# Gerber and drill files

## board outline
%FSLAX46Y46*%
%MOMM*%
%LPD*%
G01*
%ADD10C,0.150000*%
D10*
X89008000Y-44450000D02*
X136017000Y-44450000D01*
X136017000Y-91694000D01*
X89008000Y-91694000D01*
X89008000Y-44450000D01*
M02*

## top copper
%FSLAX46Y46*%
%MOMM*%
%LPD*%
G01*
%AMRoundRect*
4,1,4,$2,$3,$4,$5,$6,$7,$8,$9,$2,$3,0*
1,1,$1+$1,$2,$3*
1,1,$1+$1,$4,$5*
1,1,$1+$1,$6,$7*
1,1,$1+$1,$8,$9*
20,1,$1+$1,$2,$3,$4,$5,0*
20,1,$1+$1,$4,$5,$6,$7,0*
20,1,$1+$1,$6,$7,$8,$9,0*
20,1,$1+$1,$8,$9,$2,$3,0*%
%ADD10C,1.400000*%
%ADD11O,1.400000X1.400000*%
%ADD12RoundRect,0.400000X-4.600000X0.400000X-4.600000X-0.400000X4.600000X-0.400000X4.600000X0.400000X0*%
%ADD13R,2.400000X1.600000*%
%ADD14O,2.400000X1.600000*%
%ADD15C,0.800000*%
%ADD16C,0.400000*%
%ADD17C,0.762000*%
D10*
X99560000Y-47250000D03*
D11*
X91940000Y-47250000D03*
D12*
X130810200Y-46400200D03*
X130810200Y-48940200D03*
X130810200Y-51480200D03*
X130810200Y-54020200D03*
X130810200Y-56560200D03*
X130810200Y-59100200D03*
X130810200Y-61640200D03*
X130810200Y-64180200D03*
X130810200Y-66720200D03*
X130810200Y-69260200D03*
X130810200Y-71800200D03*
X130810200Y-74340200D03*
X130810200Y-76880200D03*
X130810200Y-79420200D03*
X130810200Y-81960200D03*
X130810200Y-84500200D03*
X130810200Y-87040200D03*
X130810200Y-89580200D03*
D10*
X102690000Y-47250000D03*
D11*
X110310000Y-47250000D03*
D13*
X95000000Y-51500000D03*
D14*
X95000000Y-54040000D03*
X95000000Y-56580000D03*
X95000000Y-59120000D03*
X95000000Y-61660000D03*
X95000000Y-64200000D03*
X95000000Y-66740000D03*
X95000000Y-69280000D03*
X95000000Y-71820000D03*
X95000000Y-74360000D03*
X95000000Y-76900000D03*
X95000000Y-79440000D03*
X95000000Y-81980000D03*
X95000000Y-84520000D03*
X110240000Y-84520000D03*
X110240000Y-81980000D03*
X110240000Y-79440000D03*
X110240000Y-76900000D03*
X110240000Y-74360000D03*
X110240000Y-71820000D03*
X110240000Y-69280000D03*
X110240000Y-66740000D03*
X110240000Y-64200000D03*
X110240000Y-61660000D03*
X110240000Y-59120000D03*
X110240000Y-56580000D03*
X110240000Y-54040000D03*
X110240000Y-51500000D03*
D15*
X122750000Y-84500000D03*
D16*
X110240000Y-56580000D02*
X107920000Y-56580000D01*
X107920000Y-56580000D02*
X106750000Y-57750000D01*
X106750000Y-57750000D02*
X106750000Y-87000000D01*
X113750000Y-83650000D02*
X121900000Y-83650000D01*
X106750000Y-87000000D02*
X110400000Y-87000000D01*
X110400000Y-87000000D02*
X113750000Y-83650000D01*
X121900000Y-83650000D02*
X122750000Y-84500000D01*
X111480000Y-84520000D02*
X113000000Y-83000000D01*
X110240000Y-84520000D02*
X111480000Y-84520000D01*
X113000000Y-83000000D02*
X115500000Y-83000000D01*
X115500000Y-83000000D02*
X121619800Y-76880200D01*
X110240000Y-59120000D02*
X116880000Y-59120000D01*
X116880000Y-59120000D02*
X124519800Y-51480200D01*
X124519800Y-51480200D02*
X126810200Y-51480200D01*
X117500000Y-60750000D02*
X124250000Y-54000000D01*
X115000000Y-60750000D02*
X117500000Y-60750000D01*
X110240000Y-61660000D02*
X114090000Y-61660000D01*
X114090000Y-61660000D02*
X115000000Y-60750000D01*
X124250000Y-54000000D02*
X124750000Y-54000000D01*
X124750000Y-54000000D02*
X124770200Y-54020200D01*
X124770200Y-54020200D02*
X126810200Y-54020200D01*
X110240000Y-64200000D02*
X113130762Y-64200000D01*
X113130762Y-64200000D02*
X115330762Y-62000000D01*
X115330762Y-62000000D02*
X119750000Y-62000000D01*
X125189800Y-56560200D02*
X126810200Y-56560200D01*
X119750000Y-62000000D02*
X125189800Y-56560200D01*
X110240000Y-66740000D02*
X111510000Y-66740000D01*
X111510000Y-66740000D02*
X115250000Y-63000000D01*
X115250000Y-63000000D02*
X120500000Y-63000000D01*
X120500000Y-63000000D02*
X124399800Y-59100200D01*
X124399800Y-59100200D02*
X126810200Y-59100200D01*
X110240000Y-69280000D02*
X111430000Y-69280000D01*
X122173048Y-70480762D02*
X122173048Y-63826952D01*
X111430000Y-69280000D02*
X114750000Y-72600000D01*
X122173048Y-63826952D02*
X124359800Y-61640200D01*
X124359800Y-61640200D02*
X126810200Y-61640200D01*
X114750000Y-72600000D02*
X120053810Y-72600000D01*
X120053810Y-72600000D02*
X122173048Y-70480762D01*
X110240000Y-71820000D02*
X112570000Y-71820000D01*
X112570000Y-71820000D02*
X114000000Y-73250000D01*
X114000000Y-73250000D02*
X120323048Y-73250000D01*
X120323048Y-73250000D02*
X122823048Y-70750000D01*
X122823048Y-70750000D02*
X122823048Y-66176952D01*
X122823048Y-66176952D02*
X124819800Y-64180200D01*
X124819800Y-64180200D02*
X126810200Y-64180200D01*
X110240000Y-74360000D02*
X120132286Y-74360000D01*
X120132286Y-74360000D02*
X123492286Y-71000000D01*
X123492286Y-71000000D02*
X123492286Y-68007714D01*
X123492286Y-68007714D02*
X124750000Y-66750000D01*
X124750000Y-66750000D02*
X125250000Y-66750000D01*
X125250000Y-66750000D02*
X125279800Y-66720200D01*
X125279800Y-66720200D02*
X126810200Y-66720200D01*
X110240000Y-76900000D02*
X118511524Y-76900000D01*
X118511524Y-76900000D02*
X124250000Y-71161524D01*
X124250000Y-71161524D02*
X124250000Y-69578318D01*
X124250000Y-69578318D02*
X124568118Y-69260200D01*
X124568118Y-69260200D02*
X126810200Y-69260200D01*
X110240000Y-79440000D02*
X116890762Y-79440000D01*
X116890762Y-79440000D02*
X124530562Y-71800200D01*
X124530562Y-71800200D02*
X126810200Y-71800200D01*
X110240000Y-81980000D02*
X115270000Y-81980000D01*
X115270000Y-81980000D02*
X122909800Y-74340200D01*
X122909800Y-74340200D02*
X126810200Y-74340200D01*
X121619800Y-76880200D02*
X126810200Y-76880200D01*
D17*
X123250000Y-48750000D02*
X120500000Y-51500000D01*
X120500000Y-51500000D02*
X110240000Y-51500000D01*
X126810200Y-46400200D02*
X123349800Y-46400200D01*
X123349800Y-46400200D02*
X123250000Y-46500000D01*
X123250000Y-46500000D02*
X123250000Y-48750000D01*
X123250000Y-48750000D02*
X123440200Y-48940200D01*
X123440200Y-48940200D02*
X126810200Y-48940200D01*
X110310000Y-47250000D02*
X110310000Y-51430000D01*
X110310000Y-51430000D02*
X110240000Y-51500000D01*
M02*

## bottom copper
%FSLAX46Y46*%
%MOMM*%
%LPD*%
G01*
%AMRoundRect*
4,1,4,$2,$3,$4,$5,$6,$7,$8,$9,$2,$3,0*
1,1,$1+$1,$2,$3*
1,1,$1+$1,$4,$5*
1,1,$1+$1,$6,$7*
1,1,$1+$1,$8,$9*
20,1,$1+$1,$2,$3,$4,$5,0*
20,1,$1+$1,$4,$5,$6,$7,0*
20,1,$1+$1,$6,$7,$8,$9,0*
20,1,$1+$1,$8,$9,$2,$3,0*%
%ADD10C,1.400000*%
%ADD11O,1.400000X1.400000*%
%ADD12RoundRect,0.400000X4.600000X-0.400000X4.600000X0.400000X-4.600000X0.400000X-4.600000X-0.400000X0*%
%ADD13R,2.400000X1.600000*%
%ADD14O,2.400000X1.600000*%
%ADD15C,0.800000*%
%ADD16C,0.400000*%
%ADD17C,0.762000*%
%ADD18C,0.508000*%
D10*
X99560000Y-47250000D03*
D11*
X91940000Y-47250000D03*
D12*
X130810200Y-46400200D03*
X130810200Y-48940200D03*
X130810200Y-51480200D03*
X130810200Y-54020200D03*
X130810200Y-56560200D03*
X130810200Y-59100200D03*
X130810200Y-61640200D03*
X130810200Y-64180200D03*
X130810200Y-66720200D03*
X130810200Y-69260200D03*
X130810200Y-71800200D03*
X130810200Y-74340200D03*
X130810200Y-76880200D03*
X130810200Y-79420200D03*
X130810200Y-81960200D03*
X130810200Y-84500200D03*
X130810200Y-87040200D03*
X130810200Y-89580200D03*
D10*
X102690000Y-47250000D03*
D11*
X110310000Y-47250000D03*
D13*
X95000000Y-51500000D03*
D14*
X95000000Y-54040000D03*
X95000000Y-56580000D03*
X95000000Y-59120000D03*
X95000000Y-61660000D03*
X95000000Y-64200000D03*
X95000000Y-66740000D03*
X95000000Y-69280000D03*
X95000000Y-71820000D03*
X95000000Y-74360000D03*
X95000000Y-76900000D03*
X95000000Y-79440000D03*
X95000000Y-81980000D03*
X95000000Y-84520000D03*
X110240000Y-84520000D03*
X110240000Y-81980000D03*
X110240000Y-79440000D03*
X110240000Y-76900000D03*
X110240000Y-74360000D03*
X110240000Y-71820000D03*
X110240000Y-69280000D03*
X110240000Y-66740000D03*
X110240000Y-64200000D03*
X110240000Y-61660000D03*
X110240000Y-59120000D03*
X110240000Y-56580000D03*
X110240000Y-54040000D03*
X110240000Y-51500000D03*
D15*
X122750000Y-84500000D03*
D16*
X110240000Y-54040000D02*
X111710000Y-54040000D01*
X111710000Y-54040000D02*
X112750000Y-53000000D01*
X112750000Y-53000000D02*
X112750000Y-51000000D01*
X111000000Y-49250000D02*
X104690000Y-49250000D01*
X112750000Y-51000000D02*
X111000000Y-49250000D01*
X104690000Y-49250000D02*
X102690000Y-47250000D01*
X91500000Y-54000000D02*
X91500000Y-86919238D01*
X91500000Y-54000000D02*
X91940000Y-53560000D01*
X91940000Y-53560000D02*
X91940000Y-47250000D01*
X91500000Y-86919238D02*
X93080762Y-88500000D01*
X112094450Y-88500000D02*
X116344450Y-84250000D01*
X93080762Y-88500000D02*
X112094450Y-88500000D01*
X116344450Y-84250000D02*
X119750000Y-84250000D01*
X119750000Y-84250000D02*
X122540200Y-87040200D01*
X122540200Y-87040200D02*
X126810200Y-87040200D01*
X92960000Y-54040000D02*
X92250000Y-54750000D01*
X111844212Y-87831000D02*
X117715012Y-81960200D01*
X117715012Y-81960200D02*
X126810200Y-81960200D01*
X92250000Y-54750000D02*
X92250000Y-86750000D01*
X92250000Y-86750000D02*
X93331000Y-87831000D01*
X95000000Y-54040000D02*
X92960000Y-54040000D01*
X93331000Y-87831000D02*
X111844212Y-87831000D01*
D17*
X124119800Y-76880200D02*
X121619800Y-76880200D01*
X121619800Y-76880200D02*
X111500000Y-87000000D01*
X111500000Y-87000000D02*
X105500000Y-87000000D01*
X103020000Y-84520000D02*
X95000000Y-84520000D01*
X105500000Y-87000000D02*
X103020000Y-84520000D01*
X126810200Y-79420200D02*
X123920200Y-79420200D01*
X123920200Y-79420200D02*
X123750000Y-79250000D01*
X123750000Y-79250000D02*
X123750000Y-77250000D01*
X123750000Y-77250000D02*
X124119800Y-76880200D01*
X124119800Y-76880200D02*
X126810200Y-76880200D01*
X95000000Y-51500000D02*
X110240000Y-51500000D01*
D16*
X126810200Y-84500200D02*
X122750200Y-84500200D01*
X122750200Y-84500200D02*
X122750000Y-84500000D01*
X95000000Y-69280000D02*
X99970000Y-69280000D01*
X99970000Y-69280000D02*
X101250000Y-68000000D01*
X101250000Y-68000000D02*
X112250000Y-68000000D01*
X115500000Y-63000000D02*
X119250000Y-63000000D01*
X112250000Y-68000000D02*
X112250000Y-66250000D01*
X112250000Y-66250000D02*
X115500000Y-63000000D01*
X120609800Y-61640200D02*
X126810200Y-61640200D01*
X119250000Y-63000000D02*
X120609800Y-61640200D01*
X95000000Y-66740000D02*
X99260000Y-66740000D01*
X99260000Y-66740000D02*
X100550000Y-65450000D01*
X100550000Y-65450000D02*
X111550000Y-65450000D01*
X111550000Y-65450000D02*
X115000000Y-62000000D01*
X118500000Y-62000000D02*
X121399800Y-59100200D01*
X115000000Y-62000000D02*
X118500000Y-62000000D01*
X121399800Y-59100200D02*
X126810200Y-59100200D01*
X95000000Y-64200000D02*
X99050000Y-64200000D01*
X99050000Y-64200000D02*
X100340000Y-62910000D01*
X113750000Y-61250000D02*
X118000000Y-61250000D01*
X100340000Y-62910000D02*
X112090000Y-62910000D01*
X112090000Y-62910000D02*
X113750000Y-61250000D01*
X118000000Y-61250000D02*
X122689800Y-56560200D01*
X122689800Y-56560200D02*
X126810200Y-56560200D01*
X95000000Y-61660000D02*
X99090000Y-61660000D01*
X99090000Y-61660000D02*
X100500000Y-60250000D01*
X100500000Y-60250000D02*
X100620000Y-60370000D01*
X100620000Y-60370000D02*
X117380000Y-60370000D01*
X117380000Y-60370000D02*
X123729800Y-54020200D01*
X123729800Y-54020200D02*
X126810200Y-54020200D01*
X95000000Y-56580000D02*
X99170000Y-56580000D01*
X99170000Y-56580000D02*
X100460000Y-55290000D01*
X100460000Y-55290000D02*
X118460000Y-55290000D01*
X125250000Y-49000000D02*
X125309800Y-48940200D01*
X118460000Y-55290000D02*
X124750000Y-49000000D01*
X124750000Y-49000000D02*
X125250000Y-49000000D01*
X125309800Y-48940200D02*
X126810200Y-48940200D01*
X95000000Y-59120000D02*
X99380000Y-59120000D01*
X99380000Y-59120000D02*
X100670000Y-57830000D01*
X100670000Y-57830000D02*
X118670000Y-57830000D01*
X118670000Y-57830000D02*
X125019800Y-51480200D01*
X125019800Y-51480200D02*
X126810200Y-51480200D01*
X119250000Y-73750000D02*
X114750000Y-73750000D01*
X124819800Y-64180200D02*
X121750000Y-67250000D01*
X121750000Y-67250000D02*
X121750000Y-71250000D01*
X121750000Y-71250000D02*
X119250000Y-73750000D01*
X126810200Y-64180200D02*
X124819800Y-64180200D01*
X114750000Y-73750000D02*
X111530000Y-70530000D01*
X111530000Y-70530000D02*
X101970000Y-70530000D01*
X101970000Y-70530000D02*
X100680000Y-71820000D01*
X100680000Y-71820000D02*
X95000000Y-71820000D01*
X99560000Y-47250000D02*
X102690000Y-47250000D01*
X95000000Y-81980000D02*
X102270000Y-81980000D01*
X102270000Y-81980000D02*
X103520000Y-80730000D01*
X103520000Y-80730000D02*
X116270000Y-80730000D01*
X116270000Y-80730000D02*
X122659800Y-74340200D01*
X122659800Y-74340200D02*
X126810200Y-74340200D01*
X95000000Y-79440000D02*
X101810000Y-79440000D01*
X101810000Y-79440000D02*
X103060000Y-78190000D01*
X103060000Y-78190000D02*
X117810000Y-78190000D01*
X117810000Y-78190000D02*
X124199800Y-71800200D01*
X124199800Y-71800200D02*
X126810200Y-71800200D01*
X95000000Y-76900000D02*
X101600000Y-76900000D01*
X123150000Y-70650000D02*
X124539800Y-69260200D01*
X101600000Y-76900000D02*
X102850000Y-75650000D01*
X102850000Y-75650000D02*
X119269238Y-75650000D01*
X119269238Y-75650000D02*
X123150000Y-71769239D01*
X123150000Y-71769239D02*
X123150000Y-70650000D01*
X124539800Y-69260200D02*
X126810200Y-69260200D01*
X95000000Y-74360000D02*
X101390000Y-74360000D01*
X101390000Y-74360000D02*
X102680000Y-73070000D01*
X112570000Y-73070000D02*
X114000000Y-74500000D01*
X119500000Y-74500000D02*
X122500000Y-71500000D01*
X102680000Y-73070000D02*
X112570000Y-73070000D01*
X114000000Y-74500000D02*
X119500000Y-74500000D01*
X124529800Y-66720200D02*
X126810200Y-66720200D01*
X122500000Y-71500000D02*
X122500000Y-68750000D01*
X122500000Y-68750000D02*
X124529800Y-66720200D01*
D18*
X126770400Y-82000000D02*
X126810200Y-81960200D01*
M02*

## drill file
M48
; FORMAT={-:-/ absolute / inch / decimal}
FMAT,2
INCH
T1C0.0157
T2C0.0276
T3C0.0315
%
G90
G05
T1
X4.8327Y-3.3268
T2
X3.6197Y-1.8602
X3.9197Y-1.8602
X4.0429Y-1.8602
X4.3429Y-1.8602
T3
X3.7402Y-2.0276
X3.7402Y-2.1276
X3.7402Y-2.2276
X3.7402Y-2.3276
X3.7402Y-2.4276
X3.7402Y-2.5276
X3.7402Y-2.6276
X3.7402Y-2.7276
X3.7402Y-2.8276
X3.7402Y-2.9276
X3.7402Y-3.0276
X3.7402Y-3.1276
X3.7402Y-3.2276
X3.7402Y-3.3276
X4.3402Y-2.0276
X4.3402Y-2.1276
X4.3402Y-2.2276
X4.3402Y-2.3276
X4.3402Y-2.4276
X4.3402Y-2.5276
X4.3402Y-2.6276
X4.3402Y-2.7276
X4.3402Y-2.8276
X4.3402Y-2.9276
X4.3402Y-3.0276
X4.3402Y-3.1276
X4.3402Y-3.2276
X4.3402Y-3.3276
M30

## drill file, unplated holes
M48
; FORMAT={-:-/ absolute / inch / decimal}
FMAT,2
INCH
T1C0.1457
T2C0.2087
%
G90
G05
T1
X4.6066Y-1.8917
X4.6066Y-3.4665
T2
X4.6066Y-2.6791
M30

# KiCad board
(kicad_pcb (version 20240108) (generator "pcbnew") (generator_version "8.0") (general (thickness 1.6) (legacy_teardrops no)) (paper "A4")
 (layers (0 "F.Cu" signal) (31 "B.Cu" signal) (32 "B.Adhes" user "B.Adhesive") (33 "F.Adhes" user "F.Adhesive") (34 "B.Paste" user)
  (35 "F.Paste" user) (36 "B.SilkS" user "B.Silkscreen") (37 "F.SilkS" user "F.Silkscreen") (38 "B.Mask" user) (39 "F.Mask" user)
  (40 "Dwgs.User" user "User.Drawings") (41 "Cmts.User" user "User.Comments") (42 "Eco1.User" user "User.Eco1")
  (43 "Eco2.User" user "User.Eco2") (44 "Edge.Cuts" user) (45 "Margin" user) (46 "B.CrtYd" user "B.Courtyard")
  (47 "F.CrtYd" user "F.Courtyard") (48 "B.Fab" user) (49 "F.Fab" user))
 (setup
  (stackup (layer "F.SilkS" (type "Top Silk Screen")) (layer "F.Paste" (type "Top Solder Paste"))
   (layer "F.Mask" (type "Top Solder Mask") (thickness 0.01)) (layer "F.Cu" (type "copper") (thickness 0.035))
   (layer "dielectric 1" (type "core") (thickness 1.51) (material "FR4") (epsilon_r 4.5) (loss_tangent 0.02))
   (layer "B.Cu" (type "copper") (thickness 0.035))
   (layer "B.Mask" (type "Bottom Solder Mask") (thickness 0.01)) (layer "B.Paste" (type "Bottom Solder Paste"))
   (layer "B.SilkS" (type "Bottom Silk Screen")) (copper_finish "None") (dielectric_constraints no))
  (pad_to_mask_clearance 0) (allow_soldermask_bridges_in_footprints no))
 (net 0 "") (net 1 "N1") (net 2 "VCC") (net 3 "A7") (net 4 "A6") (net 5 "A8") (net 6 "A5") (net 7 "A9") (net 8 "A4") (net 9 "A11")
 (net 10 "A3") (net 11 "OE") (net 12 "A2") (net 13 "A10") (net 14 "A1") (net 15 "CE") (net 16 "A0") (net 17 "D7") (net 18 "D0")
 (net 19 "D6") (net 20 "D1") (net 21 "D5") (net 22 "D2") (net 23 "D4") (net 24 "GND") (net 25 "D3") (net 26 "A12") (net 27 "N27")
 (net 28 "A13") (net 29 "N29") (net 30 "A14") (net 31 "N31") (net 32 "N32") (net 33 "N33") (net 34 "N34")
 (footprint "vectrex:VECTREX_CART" (layer "F.Cu") (at 130.8102 67.9902 -90)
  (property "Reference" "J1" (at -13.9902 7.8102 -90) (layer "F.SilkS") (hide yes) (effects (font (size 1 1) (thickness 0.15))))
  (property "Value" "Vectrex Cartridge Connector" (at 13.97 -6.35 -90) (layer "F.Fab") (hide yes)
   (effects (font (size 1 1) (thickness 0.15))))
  (pad "1" connect roundrect (at -21.59 4 90) (size 1.6 10) (drill (offset 0 4)) (layers "B.Cu" "B.Mask") (roundrect_rratio 0.25)
   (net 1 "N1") (zone_connect 2))
  (pad "2" connect roundrect (at -21.59 4 270) (size 1.6 10) (drill (offset 0 -4)) (layers "F.Cu" "F.Mask") (roundrect_rratio 0.25)
   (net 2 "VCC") (zone_connect 2))
  (pad "3" connect roundrect (at -19.05 4 90) (size 1.6 10) (drill (offset 0 4)) (layers "B.Cu" "B.Mask") (roundrect_rratio 0.25)
   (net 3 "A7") (zone_connect 2))
  (pad "4" connect roundrect (at -19.05 4 270) (size 1.6 10) (drill (offset 0 -4)) (layers "F.Cu" "F.Mask") (roundrect_rratio 0.25)
   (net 2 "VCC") (zone_connect 2))
  (pad "5" connect roundrect (at -16.51 4 90) (size 1.6 10) (drill (offset 0 4)) (layers "B.Cu" "B.Mask") (roundrect_rratio 0.25)
   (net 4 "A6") (zone_connect 2))
  (pad "6" connect roundrect (at -16.51 4 270) (size 1.6 10) (drill (offset 0 -4)) (layers "F.Cu" "F.Mask") (roundrect_rratio 0.25)
   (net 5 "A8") (zone_connect 2))
  (pad "7" connect roundrect (at -13.97 4 90) (size 1.6 10) (drill (offset 0 4)) (layers "B.Cu" "B.Mask") (roundrect_rratio 0.25)
   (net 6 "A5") (zone_connect 2))
  (pad "8" connect roundrect (at -13.97 4 270) (size 1.6 10) (drill (offset 0 -4)) (layers "F.Cu" "F.Mask") (roundrect_rratio 0.25)
   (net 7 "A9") (zone_connect 2))
  (pad "9" connect roundrect (at -11.43 4 90) (size 1.6 10) (drill (offset 0 4)) (layers "B.Cu" "B.Mask") (roundrect_rratio 0.25)
   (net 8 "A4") (zone_connect 2))
  (pad "10" connect roundrect (at -11.43 4 270) (size 1.6 10) (drill (offset 0 -4)) (layers "F.Cu" "F.Mask") (roundrect_rratio 0.25)
   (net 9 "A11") (zone_connect 2))
  (pad "11" connect roundrect (at -8.89 4 90) (size 1.6 10) (drill (offset 0 4)) (layers "B.Cu" "B.Mask") (roundrect_rratio 0.25)
   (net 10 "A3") (zone_connect 2))
  (pad "12" connect roundrect (at -8.89 4 270) (size 1.6 10) (drill (offset 0 -4)) (layers "F.Cu" "F.Mask") (roundrect_rratio 0.25)
   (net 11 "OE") (zone_connect 2))
  (pad "13" connect roundrect (at -6.35 4 90) (size 1.6 10) (drill (offset 0 4)) (layers "B.Cu" "B.Mask") (roundrect_rratio 0.25)
   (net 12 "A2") (zone_connect 2))
  (pad "14" connect roundrect (at -6.35 4 270) (size 1.6 10) (drill (offset 0 -4)) (layers "F.Cu" "F.Mask") (roundrect_rratio 0.25)
   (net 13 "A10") (zone_connect 2))
  (pad "15" connect roundrect (at -3.81 4 90) (size 1.6 10) (drill (offset 0 4)) (layers "B.Cu" "B.Mask") (roundrect_rratio 0.25)
   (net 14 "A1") (zone_connect 2))
  (pad "16" connect roundrect (at -3.81 4 270) (size 1.6 10) (drill (offset 0 -4)) (layers "F.Cu" "F.Mask") (roundrect_rratio 0.25)
   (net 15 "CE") (zone_connect 2))
  (pad "17" connect roundrect (at -1.27 4 90) (size 1.6 10) (drill (offset 0 4)) (layers "B.Cu" "B.Mask") (roundrect_rratio 0.25)
   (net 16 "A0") (zone_connect 2))
  (pad "18" connect roundrect (at -1.27 4 270) (size 1.6 10) (drill (offset 0 -4)) (layers "F.Cu" "F.Mask") (roundrect_rratio 0.25)
   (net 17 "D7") (zone_connect 2))
  (pad "19" connect roundrect (at 1.27 4 90) (size 1.6 10) (drill (offset 0 4)) (layers "B.Cu" "B.Mask") (roundrect_rratio 0.25)
   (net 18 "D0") (zone_connect 2))
  (pad "20" connect roundrect (at 1.27 4 270) (size 1.6 10) (drill (offset 0 -4)) (layers "F.Cu" "F.Mask") (roundrect_rratio 0.25)
   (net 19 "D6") (zone_connect 2))
  (pad "21" connect roundrect (at 3.81 4 90) (size 1.6 10) (drill (offset 0 4)) (layers "B.Cu" "B.Mask") (roundrect_rratio 0.25)
   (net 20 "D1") (zone_connect 2))
  (pad "22" connect roundrect (at 3.81 4 270) (size 1.6 10) (drill (offset 0 -4)) (layers "F.Cu" "F.Mask") (roundrect_rratio 0.25)
   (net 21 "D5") (zone_connect 2))
  (pad "23" connect roundrect (at 6.35 4 90) (size 1.6 10) (drill (offset 0 4)) (layers "B.Cu" "B.Mask") (roundrect_rratio 0.25)
   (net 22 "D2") (zone_connect 2))
  (pad "24" connect roundrect (at 6.35 4 270) (size 1.6 10) (drill (offset 0 -4)) (layers "F.Cu" "F.Mask") (roundrect_rratio 0.25)
   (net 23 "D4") (zone_connect 2))
  (pad "25" connect roundrect (at 8.89 4 90) (size 1.6 10) (drill (offset 0 4)) (layers "B.Cu" "B.Mask") (roundrect_rratio 0.25)
   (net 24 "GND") (zone_connect 2))
  (pad "26" connect roundrect (at 8.89 4 270) (size 1.6 10) (drill (offset 0 -4)) (layers "F.Cu" "F.Mask") (roundrect_rratio 0.25)
   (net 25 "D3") (zone_connect 2))
  (pad "27" connect roundrect (at 11.43 4 90) (size 1.6 10) (drill (offset 0 4)) (layers "B.Cu" "B.Mask") (roundrect_rratio 0.25)
   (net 24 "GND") (zone_connect 2))
  (pad "28" connect roundrect (at 11.43 4 270) (size 1.6 10) (drill (offset 0 -4)) (layers "F.Cu" "F.Mask") (roundrect_rratio 0.25)
   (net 24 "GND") (zone_connect 2))
  (pad "29" connect roundrect (at 13.97 4 90) (size 1.6 10) (drill (offset 0 4)) (layers "B.Cu" "B.Mask") (roundrect_rratio 0.25)
   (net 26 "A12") (zone_connect 2))
  (pad "30" connect roundrect (at 13.97 4 270) (size 1.6 10) (drill (offset 0 -4)) (layers "F.Cu" "F.Mask") (roundrect_rratio 0.25)
   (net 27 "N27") (zone_connect 2))
  (pad "31" connect roundrect (at 16.51 4 90) (size 1.6 10) (drill (offset 0 4)) (layers "B.Cu" "B.Mask") (roundrect_rratio 0.25)
   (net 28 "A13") (zone_connect 2))
  (pad "32" connect roundrect (at 16.51 4 270) (size 1.6 10) (drill (offset 0 -4)) (layers "F.Cu" "F.Mask") (roundrect_rratio 0.25)
   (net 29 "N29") (zone_connect 2))
  (pad "33" connect roundrect (at 19.05 4 90) (size 1.6 10) (drill (offset 0 4)) (layers "B.Cu" "B.Mask") (roundrect_rratio 0.25)
   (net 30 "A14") (zone_connect 2))
  (pad "34" connect roundrect (at 19.05 4 270) (size 1.6 10) (drill (offset 0 -4)) (layers "F.Cu" "F.Mask") (roundrect_rratio 0.25)
   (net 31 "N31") (zone_connect 2))
  (pad "35" connect roundrect (at 21.59 4 90) (size 1.6 10) (drill (offset 0 4)) (layers "B.Cu" "B.Mask") (roundrect_rratio 0.25)
   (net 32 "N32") (zone_connect 2))
  (pad "36" connect roundrect (at 21.59 4 270) (size 1.6 10) (drill (offset 0 -4)) (layers "F.Cu" "F.Mask") (roundrect_rratio 0.25)
   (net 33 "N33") (zone_connect 2)))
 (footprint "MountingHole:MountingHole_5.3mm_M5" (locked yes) (layer "F.Cu") (at 117.008 68.05)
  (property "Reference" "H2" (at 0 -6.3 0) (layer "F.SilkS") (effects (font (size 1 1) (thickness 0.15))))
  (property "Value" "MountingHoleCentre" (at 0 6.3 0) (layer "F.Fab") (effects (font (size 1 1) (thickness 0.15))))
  (pad "" np_thru_hole circle (at 0 0) (size 5.3 5.3) (drill 5.3) (layers "*.Cu" "*.Mask")))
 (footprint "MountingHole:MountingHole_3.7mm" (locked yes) (layer "F.Cu") (at 117.008 48.05)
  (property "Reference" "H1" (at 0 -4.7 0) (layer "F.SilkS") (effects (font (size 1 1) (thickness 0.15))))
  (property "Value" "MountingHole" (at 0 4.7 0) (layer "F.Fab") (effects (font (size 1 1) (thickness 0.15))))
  (pad "" np_thru_hole circle (at 0 0) (size 3.7 3.7) (drill 3.7) (layers "*.Cu" "*.Mask")))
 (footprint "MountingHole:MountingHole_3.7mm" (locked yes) (layer "F.Cu") (at 117.008 88.05)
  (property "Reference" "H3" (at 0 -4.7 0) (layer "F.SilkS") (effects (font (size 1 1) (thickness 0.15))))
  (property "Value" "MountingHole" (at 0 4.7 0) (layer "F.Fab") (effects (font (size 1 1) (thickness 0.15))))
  (pad "" np_thru_hole circle (at 0 0) (size 3.7 3.7) (drill 3.7) (layers "*.Cu" "*.Mask")))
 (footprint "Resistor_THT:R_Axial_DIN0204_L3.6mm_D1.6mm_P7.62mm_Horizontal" (layer "F.Cu") (at 99.56 47.25 180)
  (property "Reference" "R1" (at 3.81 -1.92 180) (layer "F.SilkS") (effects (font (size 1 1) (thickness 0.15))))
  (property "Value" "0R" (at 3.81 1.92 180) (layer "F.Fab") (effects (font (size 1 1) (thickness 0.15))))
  (pad "1" thru_hole circle (at 0 0 180) (size 1.4 1.4) (drill 0.7) (layers "*.Cu" "*.Mask") (remove_unused_layers no) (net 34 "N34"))
  (pad "2" thru_hole oval (at 7.62 0 180) (size 1.4 1.4) (drill 0.7) (layers "*.Cu" "*.Mask") (remove_unused_layers no) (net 30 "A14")))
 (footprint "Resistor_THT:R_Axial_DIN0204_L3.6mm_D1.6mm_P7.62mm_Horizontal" (layer "F.Cu") (at 102.69 47.25)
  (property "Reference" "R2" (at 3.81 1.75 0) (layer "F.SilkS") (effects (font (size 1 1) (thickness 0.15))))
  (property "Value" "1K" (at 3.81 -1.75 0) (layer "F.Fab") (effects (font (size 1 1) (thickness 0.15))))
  (pad "1" thru_hole circle (at 0 0) (size 1.4 1.4) (drill 0.7) (layers "*.Cu" "*.Mask") (remove_unused_layers no) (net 34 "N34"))
  (pad "2" thru_hole oval (at 7.62 0) (size 1.4 1.4) (drill 0.7) (layers "*.Cu" "*.Mask") (remove_unused_layers no) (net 2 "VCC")))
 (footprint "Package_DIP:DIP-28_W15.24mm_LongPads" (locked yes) (layer "F.Cu") (at 95 51.5)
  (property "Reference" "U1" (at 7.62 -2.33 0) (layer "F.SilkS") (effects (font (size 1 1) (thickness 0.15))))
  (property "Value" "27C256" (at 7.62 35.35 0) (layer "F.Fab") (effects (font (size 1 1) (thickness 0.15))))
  (pad "1" thru_hole rect (at 0 0) (size 2.4 1.6) (drill 0.8) (layers "*.Cu" "*.Mask") (remove_unused_layers no) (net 2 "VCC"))
  (pad "2" thru_hole oval (at 0 2.54) (size 2.4 1.6) (drill 0.8) (layers "*.Cu" "*.Mask") (remove_unused_layers no) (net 26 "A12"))
  (pad "3" thru_hole oval (at 0 5.08) (size 2.4 1.6) (drill 0.8) (layers "*.Cu" "*.Mask") (remove_unused_layers no) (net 3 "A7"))
  (pad "4" thru_hole oval (at 0 7.62) (size 2.4 1.6) (drill 0.8) (layers "*.Cu" "*.Mask") (remove_unused_layers no) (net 4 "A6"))
  (pad "5" thru_hole oval (at 0 10.16) (size 2.4 1.6) (drill 0.8) (layers "*.Cu" "*.Mask") (remove_unused_layers no) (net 6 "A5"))
  (pad "6" thru_hole oval (at 0 12.7) (size 2.4 1.6) (drill 0.8) (layers "*.Cu" "*.Mask") (remove_unused_layers no) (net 8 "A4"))
  (pad "7" thru_hole oval (at 0 15.24) (size 2.4 1.6) (drill 0.8) (layers "*.Cu" "*.Mask") (remove_unused_layers no) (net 10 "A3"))
  (pad "8" thru_hole oval (at 0 17.78) (size 2.4 1.6) (drill 0.8) (layers "*.Cu" "*.Mask") (remove_unused_layers no) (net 12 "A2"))
  (pad "9" thru_hole oval (at 0 20.32) (size 2.4 1.6) (drill 0.8) (layers "*.Cu" "*.Mask") (remove_unused_layers no) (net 14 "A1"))
  (pad "10" thru_hole oval (at 0 22.86) (size 2.4 1.6) (drill 0.8) (layers "*.Cu" "*.Mask") (remove_unused_layers no) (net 16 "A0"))
  (pad "11" thru_hole oval (at 0 25.4) (size 2.4 1.6) (drill 0.8) (layers "*.Cu" "*.Mask") (remove_unused_layers no) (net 18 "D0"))
  (pad "12" thru_hole oval (at 0 27.94) (size 2.4 1.6) (drill 0.8) (layers "*.Cu" "*.Mask") (remove_unused_layers no) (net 20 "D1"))
  (pad "13" thru_hole oval (at 0 30.48) (size 2.4 1.6) (drill 0.8) (layers "*.Cu" "*.Mask") (remove_unused_layers no) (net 22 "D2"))
  (pad "14" thru_hole oval (at 0 33.02) (size 2.4 1.6) (drill 0.8) (layers "*.Cu" "*.Mask") (remove_unused_layers no) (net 24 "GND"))
  (pad "15" thru_hole oval (at 15.24 33.02) (size 2.4 1.6) (drill 0.8) (layers "*.Cu" "*.Mask") (remove_unused_layers no) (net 25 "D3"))
  (pad "16" thru_hole oval (at 15.24 30.48) (size 2.4 1.6) (drill 0.8) (layers "*.Cu" "*.Mask") (remove_unused_layers no) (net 23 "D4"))
  (pad "17" thru_hole oval (at 15.24 27.94) (size 2.4 1.6) (drill 0.8) (layers "*.Cu" "*.Mask") (remove_unused_layers no) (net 21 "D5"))
  (pad "18" thru_hole oval (at 15.24 25.4) (size 2.4 1.6) (drill 0.8) (layers "*.Cu" "*.Mask") (remove_unused_layers no) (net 19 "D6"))
  (pad "19" thru_hole oval (at 15.24 22.86) (size 2.4 1.6) (drill 0.8) (layers "*.Cu" "*.Mask") (remove_unused_layers no) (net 17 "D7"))
  (pad "20" thru_hole oval (at 15.24 20.32) (size 2.4 1.6) (drill 0.8) (layers "*.Cu" "*.Mask") (remove_unused_layers no) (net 15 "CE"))
  (pad "21" thru_hole oval (at 15.24 17.78) (size 2.4 1.6) (drill 0.8) (layers "*.Cu" "*.Mask") (remove_unused_layers no) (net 13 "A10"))
  (pad "22" thru_hole oval (at 15.24 15.24) (size 2.4 1.6) (drill 0.8) (layers "*.Cu" "*.Mask") (remove_unused_layers no) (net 11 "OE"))
  (pad "23" thru_hole oval (at 15.24 12.7) (size 2.4 1.6) (drill 0.8) (layers "*.Cu" "*.Mask") (remove_unused_layers no) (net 9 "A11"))
  (pad "24" thru_hole oval (at 15.24 10.16) (size 2.4 1.6) (drill 0.8) (layers "*.Cu" "*.Mask") (remove_unused_layers no) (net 7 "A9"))
  (pad "25" thru_hole oval (at 15.24 7.62) (size 2.4 1.6) (drill 0.8) (layers "*.Cu" "*.Mask") (remove_unused_layers no) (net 5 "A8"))
  (pad "26" thru_hole oval (at 15.24 5.08) (size 2.4 1.6) (drill 0.8) (layers "*.Cu" "*.Mask") (remove_unused_layers no) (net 28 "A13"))
  (pad "27" thru_hole oval (at 15.24 2.54) (size 2.4 1.6) (drill 0.8) (layers "*.Cu" "*.Mask") (remove_unused_layers no) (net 34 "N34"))
  (pad "28" thru_hole oval (at 15.24 0) (size 2.4 1.6) (drill 0.8) (layers "*.Cu" "*.Mask") (remove_unused_layers no) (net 2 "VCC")))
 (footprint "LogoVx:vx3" (layer "B.Cu") (at 102.75 69.5 -90)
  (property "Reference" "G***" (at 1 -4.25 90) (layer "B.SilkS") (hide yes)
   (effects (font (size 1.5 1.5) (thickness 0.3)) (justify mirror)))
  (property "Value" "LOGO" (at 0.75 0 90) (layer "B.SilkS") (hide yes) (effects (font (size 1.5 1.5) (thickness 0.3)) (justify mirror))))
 (gr_rect (start 89.008 44.45) (end 136.017 91.694) (locked yes) (stroke (width 0.15) (type solid)) (fill none) (layer "Edge.Cuts"))
 (segment (start 123.9202 79.4202) (end 123.75 79.25) (width 0.762) (layer "B.Cu") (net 24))
 (segment (start 123.75 79.25) (end 123.75 77.25) (width 0.762) (layer "B.Cu") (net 24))
 (segment (start 111.5 87) (end 105.5 87) (width 0.762) (layer "B.Cu") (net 24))
 (segment (start 105.5 87) (end 103.02 84.52) (width 0.762) (layer "B.Cu") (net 24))
 (segment (start 124.1198 76.8802) (end 121.6198 76.8802) (width 0.762) (layer "B.Cu") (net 24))
 (segment (start 103.02 84.52) (end 95 84.52) (width 0.762) (layer "B.Cu") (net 24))
 (segment (start 123.75 77.25) (end 124.1198 76.8802) (width 0.762) (layer "B.Cu") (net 24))
 (segment (start 124.1198 76.8802) (end 126.8102 76.8802) (width 0.762) (layer "B.Cu") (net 24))
 (segment (start 126.8102 79.4202) (end 123.9202 79.4202) (width 0.762) (layer "B.Cu") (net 24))
 (segment (start 121.6198 76.8802) (end 111.5 87) (width 0.762) (layer "B.Cu") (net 24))
 (segment (start 110.31 47.25) (end 110.31 51.43) (width 0.762) (layer "F.Cu") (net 2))
 (segment (start 110.31 51.43) (end 110.24 51.5) (width 0.762) (layer "F.Cu") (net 2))
 (segment (start 123.25 46.5) (end 123.25 48.75) (width 0.762) (layer "F.Cu") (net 2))
 (segment (start 126.8102 46.4002) (end 123.3498 46.4002) (width 0.762) (layer "F.Cu") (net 2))
 (segment (start 123.25 48.75) (end 120.5 51.5) (width 0.762) (layer "F.Cu") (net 2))
 (segment (start 123.4402 48.9402) (end 126.8102 48.9402) (width 0.762) (layer "F.Cu") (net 2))
 (segment (start 123.3498 46.4002) (end 123.25 46.5) (width 0.762) (layer "F.Cu") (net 2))
 (segment (start 120.5 51.5) (end 110.24 51.5) (width 0.762) (layer "F.Cu") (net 2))
 (segment (start 123.25 48.75) (end 123.4402 48.9402) (width 0.762) (layer "F.Cu") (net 2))
 (segment (start 95 51.5) (end 110.24 51.5) (width 0.762) (layer "B.Cu") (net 2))
 (segment (start 115.5 83) (end 121.6198 76.8802) (width 0.4) (layer "F.Cu") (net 25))
 (segment (start 111.48 84.52) (end 113 83) (width 0.4) (layer "F.Cu") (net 25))
 (segment (start 110.24 84.52) (end 111.48 84.52) (width 0.4) (layer "F.Cu") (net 25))
 (segment (start 113 83) (end 115.5 83) (width 0.4) (layer "F.Cu") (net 25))
 (segment (start 121.6198 76.8802) (end 126.8102 76.8802) (width 0.4) (layer "F.Cu") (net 25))
 (segment (start 122.9098 74.3402) (end 126.8102 74.3402) (width 0.4) (layer "F.Cu") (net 23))
 (segment (start 110.24 81.98) (end 115.27 81.98) (width 0.4) (layer "F.Cu") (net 23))
 (segment (start 115.27 81.98) (end 122.9098 74.3402) (width 0.4) (layer "F.Cu") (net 23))
 (segment (start 116.890762 79.44) (end 124.530562 71.8002) (width 0.4) (layer "F.Cu") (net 21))
 (segment (start 110.24 79.44) (end 116.890762 79.44) (width 0.4) (layer "F.Cu") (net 21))
 (segment (start 124.530562 71.8002) (end 126.8102 71.8002) (width 0.4) (layer "F.Cu") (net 21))
 (segment (start 92.25 86.75) (end 93.331 87.831) (width 0.4) (layer "B.Cu") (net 26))
 (segment (start 95 54.04) (end 92.96 54.04) (width 0.4) (layer "B.Cu") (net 26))
 (segment (start 92.25 54.75) (end 92.25 86.75) (width 0.4) (layer "B.Cu") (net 26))
 (segment (start 117.715012 81.9602) (end 126.8102 81.9602) (width 0.4) (layer "B.Cu") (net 26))
 (segment (start 93.331 87.831) (end 111.844212 87.831) (width 0.4) (layer "B.Cu") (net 26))
 (segment (start 92.96 54.04) (end 92.25 54.75) (width 0.4) (layer "B.Cu") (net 26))
 (segment (start 111.844212 87.831) (end 117.715012 81.9602) (width 0.4) (layer "B.Cu") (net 26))
 (segment (start 126.7704 82) (end 126.8102 81.9602) (width 0.508) (layer "B.Cu") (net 26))
 (segment (start 124.568118 69.2602) (end 126.8102 69.2602) (width 0.4) (layer "F.Cu") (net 19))
 (segment (start 110.24 76.9) (end 118.511524 76.9) (width 0.4) (layer "F.Cu") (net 19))
 (segment (start 124.25 71.161524) (end 124.25 69.578318) (width 0.4) (layer "F.Cu") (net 19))
 (segment (start 124.25 69.578318) (end 124.568118 69.2602) (width 0.4) (layer "F.Cu") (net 19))
 (segment (start 118.511524 76.9) (end 124.25 71.161524) (width 0.4) (layer "F.Cu") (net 19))
 (segment (start 125.3098 48.9402) (end 126.8102 48.9402) (width 0.4) (layer "B.Cu") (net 3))
 (segment (start 95 56.58) (end 99.17 56.58) (width 0.4) (layer "B.Cu") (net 3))
 (segment (start 124.75 49) (end 125.25 49) (width 0.4) (layer "B.Cu") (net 3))
 (segment (start 118.46 55.29) (end 124.75 49) (width 0.4) (layer "B.Cu") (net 3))
 (segment (start 99.17 56.58) (end 100.46 55.29) (width 0.4) (layer "B.Cu") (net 3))
 (segment (start 100.46 55.29) (end 118.46 55.29) (width 0.4) (layer "B.Cu") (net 3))
 (segment (start 125.25 49) (end 125.3098 48.9402) (width 0.4) (layer "B.Cu") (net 3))
 (segment (start 123.492286 71) (end 123.492286 68.007714) (width 0.4) (layer "F.Cu") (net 17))
 (segment (start 110.24 74.36) (end 120.132286 74.36) (width 0.4) (layer "F.Cu") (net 17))
 (segment (start 124.75 66.75) (end 125.25 66.75) (width 0.4) (layer "F.Cu") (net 17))
 (segment (start 125.25 66.75) (end 125.2798 66.7202) (width 0.4) (layer "F.Cu") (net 17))
 (segment (start 123.492286 68.007714) (end 124.75 66.75) (width 0.4) (layer "F.Cu") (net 17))
 (segment (start 120.132286 74.36) (end 123.492286 71) (width 0.4) (layer "F.Cu") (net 17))
 (segment (start 125.2798 66.7202) (end 126.8102 66.7202) (width 0.4) (layer "F.Cu") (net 17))
 (segment (start 100.67 57.83) (end 118.67 57.83) (width 0.4) (layer "B.Cu") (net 4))
 (segment (start 118.67 57.83) (end 125.0198 51.4802) (width 0.4) (layer "B.Cu") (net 4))
 (segment (start 99.38 59.12) (end 100.67 57.83) (width 0.4) (layer "B.Cu") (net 4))
 (segment (start 95 59.12) (end 99.38 59.12) (width 0.4) (layer "B.Cu") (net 4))
 (segment (start 125.0198 51.4802) (end 126.8102 51.4802) (width 0.4) (layer "B.Cu") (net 4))
 (segment (start 110.24 71.82) (end 112.57 71.82) (width 0.4) (layer "F.Cu") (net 15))
 (segment (start 124.8198 64.1802) (end 126.8102 64.1802) (width 0.4) (layer "F.Cu") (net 15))
 (segment (start 112.57 71.82) (end 114 73.25) (width 0.4) (layer "F.Cu") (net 15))
 (segment (start 120.323048 73.25) (end 122.823048 70.75) (width 0.4) (layer "F.Cu") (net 15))
 (segment (start 114 73.25) (end 120.323048 73.25) (width 0.4) (layer "F.Cu") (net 15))
 (segment (start 122.823048 70.75) (end 122.823048 66.176952) (width 0.4) (layer "F.Cu") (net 15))
 (segment (start 122.823048 66.176952) (end 124.8198 64.1802) (width 0.4) (layer "F.Cu") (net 15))
 (segment (start 117.38 60.37) (end 123.7298 54.0202) (width 0.4) (layer "B.Cu") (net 6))
 (segment (start 95 61.66) (end 99.09 61.66) (width 0.4) (layer "B.Cu") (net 6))
 (segment (start 123.7298 54.0202) (end 126.8102 54.0202) (width 0.4) (layer "B.Cu") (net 6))
 (segment (start 100.5 60.25) (end 100.62 60.37) (width 0.4) (layer "B.Cu") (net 6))
 (segment (start 100.62 60.37) (end 117.38 60.37) (width 0.4) (layer "B.Cu") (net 6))
 (segment (start 99.09 61.66) (end 100.5 60.25) (width 0.4) (layer "B.Cu") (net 6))
 (segment (start 110.24 69.28) (end 111.43 69.28) (width 0.4) (layer "F.Cu") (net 13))
 (segment (start 122.173048 70.480762) (end 122.173048 63.826952) (width 0.4) (layer "F.Cu") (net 13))
 (segment (start 124.3598 61.6402) (end 126.8102 61.6402) (width 0.4) (layer "F.Cu") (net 13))
 (segment (start 122.173048 63.826952) (end 124.3598 61.6402) (width 0.4) (layer "F.Cu") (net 13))
 (segment (start 114.75 72.6) (end 120.05381 72.6) (width 0.4) (layer "F.Cu") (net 13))
 (segment (start 120.05381 72.6) (end 122.173048 70.480762) (width 0.4) (layer "F.Cu") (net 13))
 (segment (start 111.43 69.28) (end 114.75 72.6) (width 0.4) (layer "F.Cu") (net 13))
 (segment (start 122.6898 56.5602) (end 126.8102 56.5602) (width 0.4) (layer "B.Cu") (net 8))
 (segment (start 99.05 64.2) (end 100.34 62.91) (width 0.4) (layer "B.Cu") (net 8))
 (segment (start 113.75 61.25) (end 118 61.25) (width 0.4) (layer "B.Cu") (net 8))
 (segment (start 95 64.2) (end 99.05 64.2) (width 0.4) (layer "B.Cu") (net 8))
 (segment (start 118 61.25) (end 122.6898 56.5602) (width 0.4) (layer "B.Cu") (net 8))
 (segment (start 100.34 62.91) (end 112.09 62.91) (width 0.4) (layer "B.Cu") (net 8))
 (segment (start 112.09 62.91) (end 113.75 61.25) (width 0.4) (layer "B.Cu") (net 8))
 (segment (start 111.51 66.74) (end 115.25 63) (width 0.4) (layer "F.Cu") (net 11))
 (segment (start 110.24 66.74) (end 111.51 66.74) (width 0.4) (layer "F.Cu") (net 11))
 (segment (start 120.5 63) (end 124.3998 59.1002) (width 0.4) (layer "F.Cu") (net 11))
 (segment (start 115.25 63) (end 120.5 63) (width 0.4) (layer "F.Cu") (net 11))
 (segment (start 124.3998 59.1002) (end 126.8102 59.1002) (width 0.4) (layer "F.Cu") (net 11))
 (segment (start 111.55 65.45) (end 115 62) (width 0.4) (layer "B.Cu") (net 10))
 (segment (start 99.26 66.74) (end 100.55 65.45) (width 0.4) (layer "B.Cu") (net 10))
 (segment (start 115 62) (end 118.5 62) (width 0.4) (layer "B.Cu") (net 10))
 (segment (start 118.5 62) (end 121.3998 59.1002) (width 0.4) (layer "B.Cu") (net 10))
 (segment (start 100.55 65.45) (end 111.55 65.45) (width 0.4) (layer "B.Cu") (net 10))
 (segment (start 121.3998 59.1002) (end 126.8102 59.1002) (width 0.4) (layer "B.Cu") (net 10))
 (segment (start 95 66.74) (end 99.26 66.74) (width 0.4) (layer "B.Cu") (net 10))
 (segment (start 125.1898 56.5602) (end 126.8102 56.5602) (width 0.4) (layer "F.Cu") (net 9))
 (segment (start 119.75 62) (end 125.1898 56.5602) (width 0.4) (layer "F.Cu") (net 9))
 (segment (start 110.24 64.2) (end 113.130762 64.2) (width 0.4) (layer "F.Cu") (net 9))
 (segment (start 113.130762 64.2) (end 115.330762 62) (width 0.4) (layer "F.Cu") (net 9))
 (segment (start 115.330762 62) (end 119.75 62) (width 0.4) (layer "F.Cu") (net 9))
 (segment (start 101.25 68) (end 112.25 68) (width 0.4) (layer "B.Cu") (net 12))
 (segment (start 119.25 63) (end 120.6098 61.6402) (width 0.4) (layer "B.Cu") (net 12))
 (segment (start 115.5 63) (end 119.25 63) (width 0.4) (layer "B.Cu") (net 12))
 (segment (start 112.25 66.25) (end 115.5 63) (width 0.4) (layer "B.Cu") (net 12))
 (segment (start 120.6098 61.6402) (end 126.8102 61.6402) (width 0.4) (layer "B.Cu") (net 12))
 (segment (start 95 69.28) (end 99.97 69.28) (width 0.4) (layer "B.Cu") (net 12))
 (segment (start 112.25 68) (end 112.25 66.25) (width 0.4) (layer "B.Cu") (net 12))
 (segment (start 99.97 69.28) (end 101.25 68) (width 0.4) (layer "B.Cu") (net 12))
 (segment (start 114.09 61.66) (end 115 60.75) (width 0.4) (layer "F.Cu") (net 7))
 (segment (start 110.24 61.66) (end 114.09 61.66) (width 0.4) (layer "F.Cu") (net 7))
 (segment (start 124.7702 54.0202) (end 126.8102 54.0202) (width 0.4) (layer "F.Cu") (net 7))
 (segment (start 124.25 54) (end 124.75 54) (width 0.4) (layer "F.Cu") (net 7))
 (segment (start 124.75 54) (end 124.7702 54.0202) (width 0.4) (layer "F.Cu") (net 7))
 (segment (start 117.5 60.75) (end 124.25 54) (width 0.4) (layer "F.Cu") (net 7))
 (segment (start 115 60.75) (end 117.5 60.75) (width 0.4) (layer "F.Cu") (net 7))
 (segment (start 101.97 70.53) (end 100.68 71.82) (width 0.4) (layer "B.Cu") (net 14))
 (segment (start 121.75 67.25) (end 121.75 71.25) (width 0.4) (layer "B.Cu") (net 14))
 (segment (start 114.75 73.75) (end 111.53 70.53) (width 0.4) (layer "B.Cu") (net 14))
 (segment (start 121.75 71.25) (end 119.25 73.75) (width 0.4) (layer "B.Cu") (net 14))
 (segment (start 124.8198 64.1802) (end 121.75 67.25) (width 0.4) (layer "B.Cu") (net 14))
 (segment (start 100.68 71.82) (end 95 71.82) (width 0.4) (layer "B.Cu") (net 14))
 (segment (start 119.25 73.75) (end 114.75 73.75) (width 0.4) (layer "B.Cu") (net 14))
 (segment (start 111.53 70.53) (end 101.97 70.53) (width 0.4) (layer "B.Cu") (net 14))
 (segment (start 126.8102 64.1802) (end 124.8198 64.1802) (width 0.4) (layer "B.Cu") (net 14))
 (segment (start 116.88 59.12) (end 124.5198 51.4802) (width 0.4) (layer "F.Cu") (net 5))
 (segment (start 124.5198 51.4802) (end 126.8102 51.4802) (width 0.4) (layer "F.Cu") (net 5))
 (segment (start 110.24 59.12) (end 116.88 59.12) (width 0.4) (layer "F.Cu") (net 5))
 (segment (start 102.68 73.07) (end 112.57 73.07) (width 0.4) (layer "B.Cu") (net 16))
 (segment (start 124.5298 66.7202) (end 126.8102 66.7202) (width 0.4) (layer "B.Cu") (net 16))
 (segment (start 122.5 71.5) (end 122.5 68.75) (width 0.4) (layer "B.Cu") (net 16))
 (segment (start 112.57 73.07) (end 114 74.5) (width 0.4) (layer "B.Cu") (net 16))
 (segment (start 122.5 68.75) (end 124.5298 66.7202) (width 0.4) (layer "B.Cu") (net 16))
 (segment (start 101.39 74.36) (end 102.68 73.07) (width 0.4) (layer "B.Cu") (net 16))
 (segment (start 95 74.36) (end 101.39 74.36) (width 0.4) (layer "B.Cu") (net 16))
 (segment (start 114 74.5) (end 119.5 74.5) (width 0.4) (layer "B.Cu") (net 16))
 (segment (start 119.5 74.5) (end 122.5 71.5) (width 0.4) (layer "B.Cu") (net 16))
 (segment (start 124.5398 69.2602) (end 126.8102 69.2602) (width 0.4) (layer "B.Cu") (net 18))
 (segment (start 123.15 71.769239) (end 123.15 70.65) (width 0.4) (layer "B.Cu") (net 18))
 (segment (start 95 76.9) (end 101.6 76.9) (width 0.4) (layer "B.Cu") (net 18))
 (segment (start 119.269238 75.65) (end 123.15 71.769239) (width 0.4) (layer "B.Cu") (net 18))
 (segment (start 102.85 75.65) (end 119.269238 75.65) (width 0.4) (layer "B.Cu") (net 18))
 (segment (start 123.15 70.65) (end 124.5398 69.2602) (width 0.4) (layer "B.Cu") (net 18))
 (segment (start 101.6 76.9) (end 102.85 75.65) (width 0.4) (layer "B.Cu") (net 18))
 (segment (start 124.1998 71.8002) (end 126.8102 71.8002) (width 0.4) (layer "B.Cu") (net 20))
 (segment (start 95 79.44) (end 101.81 79.44) (width 0.4) (layer "B.Cu") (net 20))
 (segment (start 103.06 78.19) (end 117.81 78.19) (width 0.4) (layer "B.Cu") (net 20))
 (segment (start 117.81 78.19) (end 124.1998 71.8002) (width 0.4) (layer "B.Cu") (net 20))
 (segment (start 101.81 79.44) (end 103.06 78.19) (width 0.4) (layer "B.Cu") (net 20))
 (segment (start 102.27 81.98) (end 103.52 80.73) (width 0.4) (layer "B.Cu") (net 22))
 (segment (start 116.27 80.73) (end 122.6598 74.3402) (width 0.4) (layer "B.Cu") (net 22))
 (segment (start 103.52 80.73) (end 116.27 80.73) (width 0.4) (layer "B.Cu") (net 22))
 (segment (start 95 81.98) (end 102.27 81.98) (width 0.4) (layer "B.Cu") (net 22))
 (segment (start 122.6598 74.3402) (end 126.8102 74.3402) (width 0.4) (layer "B.Cu") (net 22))
 (segment (start 119.75 84.25) (end 122.5402 87.0402) (width 0.4) (layer "B.Cu") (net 30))
 (segment (start 112.09445 88.5) (end 116.34445 84.25) (width 0.4) (layer "B.Cu") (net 30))
 (segment (start 91.5 86.919238) (end 93.080762 88.5) (width 0.4) (layer "B.Cu") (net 30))
 (segment (start 91.5 54) (end 91.94 53.56) (width 0.4) (layer "B.Cu") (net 30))
 (segment (start 91.5 54) (end 91.5 86.919238) (width 0.4) (layer "B.Cu") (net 30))
 (segment (start 116.34445 84.25) (end 119.75 84.25) (width 0.4) (layer "B.Cu") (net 30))
 (segment (start 93.080762 88.5) (end 112.09445 88.5) (width 0.4) (layer "B.Cu") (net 30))
 (segment (start 122.5402 87.0402) (end 126.8102 87.0402) (width 0.4) (layer "B.Cu") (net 30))
 (segment (start 91.94 53.56) (end 91.94 47.25) (width 0.4) (layer "B.Cu") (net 30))
 (segment (start 107.92 56.58) (end 106.75 57.75) (width 0.4) (layer "F.Cu") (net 28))
 (segment (start 110.24 56.58) (end 107.92 56.58) (width 0.4) (layer "F.Cu") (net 28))
 (segment (start 113.75 83.65) (end 121.9 83.65) (width 0.4) (layer "F.Cu") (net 28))
 (segment (start 106.75 57.75) (end 106.75 87) (width 0.4) (layer "F.Cu") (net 28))
 (segment (start 121.9 83.65) (end 122.75 84.5) (width 0.4) (layer "F.Cu") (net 28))
 (segment (start 106.75 87) (end 110.4 87) (width 0.4) (layer "F.Cu") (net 28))
 (segment (start 110.4 87) (end 113.75 83.65) (width 0.4) (layer "F.Cu") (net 28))
 (via (at 122.75 84.5) (size 0.8) (drill 0.4) (layers "F.Cu" "B.Cu") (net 28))
 (segment (start 122.7502 84.5002) (end 122.75 84.5) (width 0.4) (layer "B.Cu") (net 28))
 (segment (start 126.8102 84.5002) (end 122.7502 84.5002) (width 0.4) (layer "B.Cu") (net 28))
 (segment (start 111 49.25) (end 104.69 49.25) (width 0.4) (layer "B.Cu") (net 34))
 (segment (start 104.69 49.25) (end 102.69 47.25) (width 0.4) (layer "B.Cu") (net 34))
 (segment (start 111.71 54.04) (end 112.75 53) (width 0.4) (layer "B.Cu") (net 34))
 (segment (start 112.75 53) (end 112.75 51) (width 0.4) (layer "B.Cu") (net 34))
 (segment (start 110.24 54.04) (end 111.71 54.04) (width 0.4) (layer "B.Cu") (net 34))
 (segment (start 99.56 47.25) (end 102.69 47.25) (width 0.4) (layer "B.Cu") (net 34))
 (segment (start 112.75 51) (end 111 49.25) (width 0.4) (layer "B.Cu") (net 34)))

